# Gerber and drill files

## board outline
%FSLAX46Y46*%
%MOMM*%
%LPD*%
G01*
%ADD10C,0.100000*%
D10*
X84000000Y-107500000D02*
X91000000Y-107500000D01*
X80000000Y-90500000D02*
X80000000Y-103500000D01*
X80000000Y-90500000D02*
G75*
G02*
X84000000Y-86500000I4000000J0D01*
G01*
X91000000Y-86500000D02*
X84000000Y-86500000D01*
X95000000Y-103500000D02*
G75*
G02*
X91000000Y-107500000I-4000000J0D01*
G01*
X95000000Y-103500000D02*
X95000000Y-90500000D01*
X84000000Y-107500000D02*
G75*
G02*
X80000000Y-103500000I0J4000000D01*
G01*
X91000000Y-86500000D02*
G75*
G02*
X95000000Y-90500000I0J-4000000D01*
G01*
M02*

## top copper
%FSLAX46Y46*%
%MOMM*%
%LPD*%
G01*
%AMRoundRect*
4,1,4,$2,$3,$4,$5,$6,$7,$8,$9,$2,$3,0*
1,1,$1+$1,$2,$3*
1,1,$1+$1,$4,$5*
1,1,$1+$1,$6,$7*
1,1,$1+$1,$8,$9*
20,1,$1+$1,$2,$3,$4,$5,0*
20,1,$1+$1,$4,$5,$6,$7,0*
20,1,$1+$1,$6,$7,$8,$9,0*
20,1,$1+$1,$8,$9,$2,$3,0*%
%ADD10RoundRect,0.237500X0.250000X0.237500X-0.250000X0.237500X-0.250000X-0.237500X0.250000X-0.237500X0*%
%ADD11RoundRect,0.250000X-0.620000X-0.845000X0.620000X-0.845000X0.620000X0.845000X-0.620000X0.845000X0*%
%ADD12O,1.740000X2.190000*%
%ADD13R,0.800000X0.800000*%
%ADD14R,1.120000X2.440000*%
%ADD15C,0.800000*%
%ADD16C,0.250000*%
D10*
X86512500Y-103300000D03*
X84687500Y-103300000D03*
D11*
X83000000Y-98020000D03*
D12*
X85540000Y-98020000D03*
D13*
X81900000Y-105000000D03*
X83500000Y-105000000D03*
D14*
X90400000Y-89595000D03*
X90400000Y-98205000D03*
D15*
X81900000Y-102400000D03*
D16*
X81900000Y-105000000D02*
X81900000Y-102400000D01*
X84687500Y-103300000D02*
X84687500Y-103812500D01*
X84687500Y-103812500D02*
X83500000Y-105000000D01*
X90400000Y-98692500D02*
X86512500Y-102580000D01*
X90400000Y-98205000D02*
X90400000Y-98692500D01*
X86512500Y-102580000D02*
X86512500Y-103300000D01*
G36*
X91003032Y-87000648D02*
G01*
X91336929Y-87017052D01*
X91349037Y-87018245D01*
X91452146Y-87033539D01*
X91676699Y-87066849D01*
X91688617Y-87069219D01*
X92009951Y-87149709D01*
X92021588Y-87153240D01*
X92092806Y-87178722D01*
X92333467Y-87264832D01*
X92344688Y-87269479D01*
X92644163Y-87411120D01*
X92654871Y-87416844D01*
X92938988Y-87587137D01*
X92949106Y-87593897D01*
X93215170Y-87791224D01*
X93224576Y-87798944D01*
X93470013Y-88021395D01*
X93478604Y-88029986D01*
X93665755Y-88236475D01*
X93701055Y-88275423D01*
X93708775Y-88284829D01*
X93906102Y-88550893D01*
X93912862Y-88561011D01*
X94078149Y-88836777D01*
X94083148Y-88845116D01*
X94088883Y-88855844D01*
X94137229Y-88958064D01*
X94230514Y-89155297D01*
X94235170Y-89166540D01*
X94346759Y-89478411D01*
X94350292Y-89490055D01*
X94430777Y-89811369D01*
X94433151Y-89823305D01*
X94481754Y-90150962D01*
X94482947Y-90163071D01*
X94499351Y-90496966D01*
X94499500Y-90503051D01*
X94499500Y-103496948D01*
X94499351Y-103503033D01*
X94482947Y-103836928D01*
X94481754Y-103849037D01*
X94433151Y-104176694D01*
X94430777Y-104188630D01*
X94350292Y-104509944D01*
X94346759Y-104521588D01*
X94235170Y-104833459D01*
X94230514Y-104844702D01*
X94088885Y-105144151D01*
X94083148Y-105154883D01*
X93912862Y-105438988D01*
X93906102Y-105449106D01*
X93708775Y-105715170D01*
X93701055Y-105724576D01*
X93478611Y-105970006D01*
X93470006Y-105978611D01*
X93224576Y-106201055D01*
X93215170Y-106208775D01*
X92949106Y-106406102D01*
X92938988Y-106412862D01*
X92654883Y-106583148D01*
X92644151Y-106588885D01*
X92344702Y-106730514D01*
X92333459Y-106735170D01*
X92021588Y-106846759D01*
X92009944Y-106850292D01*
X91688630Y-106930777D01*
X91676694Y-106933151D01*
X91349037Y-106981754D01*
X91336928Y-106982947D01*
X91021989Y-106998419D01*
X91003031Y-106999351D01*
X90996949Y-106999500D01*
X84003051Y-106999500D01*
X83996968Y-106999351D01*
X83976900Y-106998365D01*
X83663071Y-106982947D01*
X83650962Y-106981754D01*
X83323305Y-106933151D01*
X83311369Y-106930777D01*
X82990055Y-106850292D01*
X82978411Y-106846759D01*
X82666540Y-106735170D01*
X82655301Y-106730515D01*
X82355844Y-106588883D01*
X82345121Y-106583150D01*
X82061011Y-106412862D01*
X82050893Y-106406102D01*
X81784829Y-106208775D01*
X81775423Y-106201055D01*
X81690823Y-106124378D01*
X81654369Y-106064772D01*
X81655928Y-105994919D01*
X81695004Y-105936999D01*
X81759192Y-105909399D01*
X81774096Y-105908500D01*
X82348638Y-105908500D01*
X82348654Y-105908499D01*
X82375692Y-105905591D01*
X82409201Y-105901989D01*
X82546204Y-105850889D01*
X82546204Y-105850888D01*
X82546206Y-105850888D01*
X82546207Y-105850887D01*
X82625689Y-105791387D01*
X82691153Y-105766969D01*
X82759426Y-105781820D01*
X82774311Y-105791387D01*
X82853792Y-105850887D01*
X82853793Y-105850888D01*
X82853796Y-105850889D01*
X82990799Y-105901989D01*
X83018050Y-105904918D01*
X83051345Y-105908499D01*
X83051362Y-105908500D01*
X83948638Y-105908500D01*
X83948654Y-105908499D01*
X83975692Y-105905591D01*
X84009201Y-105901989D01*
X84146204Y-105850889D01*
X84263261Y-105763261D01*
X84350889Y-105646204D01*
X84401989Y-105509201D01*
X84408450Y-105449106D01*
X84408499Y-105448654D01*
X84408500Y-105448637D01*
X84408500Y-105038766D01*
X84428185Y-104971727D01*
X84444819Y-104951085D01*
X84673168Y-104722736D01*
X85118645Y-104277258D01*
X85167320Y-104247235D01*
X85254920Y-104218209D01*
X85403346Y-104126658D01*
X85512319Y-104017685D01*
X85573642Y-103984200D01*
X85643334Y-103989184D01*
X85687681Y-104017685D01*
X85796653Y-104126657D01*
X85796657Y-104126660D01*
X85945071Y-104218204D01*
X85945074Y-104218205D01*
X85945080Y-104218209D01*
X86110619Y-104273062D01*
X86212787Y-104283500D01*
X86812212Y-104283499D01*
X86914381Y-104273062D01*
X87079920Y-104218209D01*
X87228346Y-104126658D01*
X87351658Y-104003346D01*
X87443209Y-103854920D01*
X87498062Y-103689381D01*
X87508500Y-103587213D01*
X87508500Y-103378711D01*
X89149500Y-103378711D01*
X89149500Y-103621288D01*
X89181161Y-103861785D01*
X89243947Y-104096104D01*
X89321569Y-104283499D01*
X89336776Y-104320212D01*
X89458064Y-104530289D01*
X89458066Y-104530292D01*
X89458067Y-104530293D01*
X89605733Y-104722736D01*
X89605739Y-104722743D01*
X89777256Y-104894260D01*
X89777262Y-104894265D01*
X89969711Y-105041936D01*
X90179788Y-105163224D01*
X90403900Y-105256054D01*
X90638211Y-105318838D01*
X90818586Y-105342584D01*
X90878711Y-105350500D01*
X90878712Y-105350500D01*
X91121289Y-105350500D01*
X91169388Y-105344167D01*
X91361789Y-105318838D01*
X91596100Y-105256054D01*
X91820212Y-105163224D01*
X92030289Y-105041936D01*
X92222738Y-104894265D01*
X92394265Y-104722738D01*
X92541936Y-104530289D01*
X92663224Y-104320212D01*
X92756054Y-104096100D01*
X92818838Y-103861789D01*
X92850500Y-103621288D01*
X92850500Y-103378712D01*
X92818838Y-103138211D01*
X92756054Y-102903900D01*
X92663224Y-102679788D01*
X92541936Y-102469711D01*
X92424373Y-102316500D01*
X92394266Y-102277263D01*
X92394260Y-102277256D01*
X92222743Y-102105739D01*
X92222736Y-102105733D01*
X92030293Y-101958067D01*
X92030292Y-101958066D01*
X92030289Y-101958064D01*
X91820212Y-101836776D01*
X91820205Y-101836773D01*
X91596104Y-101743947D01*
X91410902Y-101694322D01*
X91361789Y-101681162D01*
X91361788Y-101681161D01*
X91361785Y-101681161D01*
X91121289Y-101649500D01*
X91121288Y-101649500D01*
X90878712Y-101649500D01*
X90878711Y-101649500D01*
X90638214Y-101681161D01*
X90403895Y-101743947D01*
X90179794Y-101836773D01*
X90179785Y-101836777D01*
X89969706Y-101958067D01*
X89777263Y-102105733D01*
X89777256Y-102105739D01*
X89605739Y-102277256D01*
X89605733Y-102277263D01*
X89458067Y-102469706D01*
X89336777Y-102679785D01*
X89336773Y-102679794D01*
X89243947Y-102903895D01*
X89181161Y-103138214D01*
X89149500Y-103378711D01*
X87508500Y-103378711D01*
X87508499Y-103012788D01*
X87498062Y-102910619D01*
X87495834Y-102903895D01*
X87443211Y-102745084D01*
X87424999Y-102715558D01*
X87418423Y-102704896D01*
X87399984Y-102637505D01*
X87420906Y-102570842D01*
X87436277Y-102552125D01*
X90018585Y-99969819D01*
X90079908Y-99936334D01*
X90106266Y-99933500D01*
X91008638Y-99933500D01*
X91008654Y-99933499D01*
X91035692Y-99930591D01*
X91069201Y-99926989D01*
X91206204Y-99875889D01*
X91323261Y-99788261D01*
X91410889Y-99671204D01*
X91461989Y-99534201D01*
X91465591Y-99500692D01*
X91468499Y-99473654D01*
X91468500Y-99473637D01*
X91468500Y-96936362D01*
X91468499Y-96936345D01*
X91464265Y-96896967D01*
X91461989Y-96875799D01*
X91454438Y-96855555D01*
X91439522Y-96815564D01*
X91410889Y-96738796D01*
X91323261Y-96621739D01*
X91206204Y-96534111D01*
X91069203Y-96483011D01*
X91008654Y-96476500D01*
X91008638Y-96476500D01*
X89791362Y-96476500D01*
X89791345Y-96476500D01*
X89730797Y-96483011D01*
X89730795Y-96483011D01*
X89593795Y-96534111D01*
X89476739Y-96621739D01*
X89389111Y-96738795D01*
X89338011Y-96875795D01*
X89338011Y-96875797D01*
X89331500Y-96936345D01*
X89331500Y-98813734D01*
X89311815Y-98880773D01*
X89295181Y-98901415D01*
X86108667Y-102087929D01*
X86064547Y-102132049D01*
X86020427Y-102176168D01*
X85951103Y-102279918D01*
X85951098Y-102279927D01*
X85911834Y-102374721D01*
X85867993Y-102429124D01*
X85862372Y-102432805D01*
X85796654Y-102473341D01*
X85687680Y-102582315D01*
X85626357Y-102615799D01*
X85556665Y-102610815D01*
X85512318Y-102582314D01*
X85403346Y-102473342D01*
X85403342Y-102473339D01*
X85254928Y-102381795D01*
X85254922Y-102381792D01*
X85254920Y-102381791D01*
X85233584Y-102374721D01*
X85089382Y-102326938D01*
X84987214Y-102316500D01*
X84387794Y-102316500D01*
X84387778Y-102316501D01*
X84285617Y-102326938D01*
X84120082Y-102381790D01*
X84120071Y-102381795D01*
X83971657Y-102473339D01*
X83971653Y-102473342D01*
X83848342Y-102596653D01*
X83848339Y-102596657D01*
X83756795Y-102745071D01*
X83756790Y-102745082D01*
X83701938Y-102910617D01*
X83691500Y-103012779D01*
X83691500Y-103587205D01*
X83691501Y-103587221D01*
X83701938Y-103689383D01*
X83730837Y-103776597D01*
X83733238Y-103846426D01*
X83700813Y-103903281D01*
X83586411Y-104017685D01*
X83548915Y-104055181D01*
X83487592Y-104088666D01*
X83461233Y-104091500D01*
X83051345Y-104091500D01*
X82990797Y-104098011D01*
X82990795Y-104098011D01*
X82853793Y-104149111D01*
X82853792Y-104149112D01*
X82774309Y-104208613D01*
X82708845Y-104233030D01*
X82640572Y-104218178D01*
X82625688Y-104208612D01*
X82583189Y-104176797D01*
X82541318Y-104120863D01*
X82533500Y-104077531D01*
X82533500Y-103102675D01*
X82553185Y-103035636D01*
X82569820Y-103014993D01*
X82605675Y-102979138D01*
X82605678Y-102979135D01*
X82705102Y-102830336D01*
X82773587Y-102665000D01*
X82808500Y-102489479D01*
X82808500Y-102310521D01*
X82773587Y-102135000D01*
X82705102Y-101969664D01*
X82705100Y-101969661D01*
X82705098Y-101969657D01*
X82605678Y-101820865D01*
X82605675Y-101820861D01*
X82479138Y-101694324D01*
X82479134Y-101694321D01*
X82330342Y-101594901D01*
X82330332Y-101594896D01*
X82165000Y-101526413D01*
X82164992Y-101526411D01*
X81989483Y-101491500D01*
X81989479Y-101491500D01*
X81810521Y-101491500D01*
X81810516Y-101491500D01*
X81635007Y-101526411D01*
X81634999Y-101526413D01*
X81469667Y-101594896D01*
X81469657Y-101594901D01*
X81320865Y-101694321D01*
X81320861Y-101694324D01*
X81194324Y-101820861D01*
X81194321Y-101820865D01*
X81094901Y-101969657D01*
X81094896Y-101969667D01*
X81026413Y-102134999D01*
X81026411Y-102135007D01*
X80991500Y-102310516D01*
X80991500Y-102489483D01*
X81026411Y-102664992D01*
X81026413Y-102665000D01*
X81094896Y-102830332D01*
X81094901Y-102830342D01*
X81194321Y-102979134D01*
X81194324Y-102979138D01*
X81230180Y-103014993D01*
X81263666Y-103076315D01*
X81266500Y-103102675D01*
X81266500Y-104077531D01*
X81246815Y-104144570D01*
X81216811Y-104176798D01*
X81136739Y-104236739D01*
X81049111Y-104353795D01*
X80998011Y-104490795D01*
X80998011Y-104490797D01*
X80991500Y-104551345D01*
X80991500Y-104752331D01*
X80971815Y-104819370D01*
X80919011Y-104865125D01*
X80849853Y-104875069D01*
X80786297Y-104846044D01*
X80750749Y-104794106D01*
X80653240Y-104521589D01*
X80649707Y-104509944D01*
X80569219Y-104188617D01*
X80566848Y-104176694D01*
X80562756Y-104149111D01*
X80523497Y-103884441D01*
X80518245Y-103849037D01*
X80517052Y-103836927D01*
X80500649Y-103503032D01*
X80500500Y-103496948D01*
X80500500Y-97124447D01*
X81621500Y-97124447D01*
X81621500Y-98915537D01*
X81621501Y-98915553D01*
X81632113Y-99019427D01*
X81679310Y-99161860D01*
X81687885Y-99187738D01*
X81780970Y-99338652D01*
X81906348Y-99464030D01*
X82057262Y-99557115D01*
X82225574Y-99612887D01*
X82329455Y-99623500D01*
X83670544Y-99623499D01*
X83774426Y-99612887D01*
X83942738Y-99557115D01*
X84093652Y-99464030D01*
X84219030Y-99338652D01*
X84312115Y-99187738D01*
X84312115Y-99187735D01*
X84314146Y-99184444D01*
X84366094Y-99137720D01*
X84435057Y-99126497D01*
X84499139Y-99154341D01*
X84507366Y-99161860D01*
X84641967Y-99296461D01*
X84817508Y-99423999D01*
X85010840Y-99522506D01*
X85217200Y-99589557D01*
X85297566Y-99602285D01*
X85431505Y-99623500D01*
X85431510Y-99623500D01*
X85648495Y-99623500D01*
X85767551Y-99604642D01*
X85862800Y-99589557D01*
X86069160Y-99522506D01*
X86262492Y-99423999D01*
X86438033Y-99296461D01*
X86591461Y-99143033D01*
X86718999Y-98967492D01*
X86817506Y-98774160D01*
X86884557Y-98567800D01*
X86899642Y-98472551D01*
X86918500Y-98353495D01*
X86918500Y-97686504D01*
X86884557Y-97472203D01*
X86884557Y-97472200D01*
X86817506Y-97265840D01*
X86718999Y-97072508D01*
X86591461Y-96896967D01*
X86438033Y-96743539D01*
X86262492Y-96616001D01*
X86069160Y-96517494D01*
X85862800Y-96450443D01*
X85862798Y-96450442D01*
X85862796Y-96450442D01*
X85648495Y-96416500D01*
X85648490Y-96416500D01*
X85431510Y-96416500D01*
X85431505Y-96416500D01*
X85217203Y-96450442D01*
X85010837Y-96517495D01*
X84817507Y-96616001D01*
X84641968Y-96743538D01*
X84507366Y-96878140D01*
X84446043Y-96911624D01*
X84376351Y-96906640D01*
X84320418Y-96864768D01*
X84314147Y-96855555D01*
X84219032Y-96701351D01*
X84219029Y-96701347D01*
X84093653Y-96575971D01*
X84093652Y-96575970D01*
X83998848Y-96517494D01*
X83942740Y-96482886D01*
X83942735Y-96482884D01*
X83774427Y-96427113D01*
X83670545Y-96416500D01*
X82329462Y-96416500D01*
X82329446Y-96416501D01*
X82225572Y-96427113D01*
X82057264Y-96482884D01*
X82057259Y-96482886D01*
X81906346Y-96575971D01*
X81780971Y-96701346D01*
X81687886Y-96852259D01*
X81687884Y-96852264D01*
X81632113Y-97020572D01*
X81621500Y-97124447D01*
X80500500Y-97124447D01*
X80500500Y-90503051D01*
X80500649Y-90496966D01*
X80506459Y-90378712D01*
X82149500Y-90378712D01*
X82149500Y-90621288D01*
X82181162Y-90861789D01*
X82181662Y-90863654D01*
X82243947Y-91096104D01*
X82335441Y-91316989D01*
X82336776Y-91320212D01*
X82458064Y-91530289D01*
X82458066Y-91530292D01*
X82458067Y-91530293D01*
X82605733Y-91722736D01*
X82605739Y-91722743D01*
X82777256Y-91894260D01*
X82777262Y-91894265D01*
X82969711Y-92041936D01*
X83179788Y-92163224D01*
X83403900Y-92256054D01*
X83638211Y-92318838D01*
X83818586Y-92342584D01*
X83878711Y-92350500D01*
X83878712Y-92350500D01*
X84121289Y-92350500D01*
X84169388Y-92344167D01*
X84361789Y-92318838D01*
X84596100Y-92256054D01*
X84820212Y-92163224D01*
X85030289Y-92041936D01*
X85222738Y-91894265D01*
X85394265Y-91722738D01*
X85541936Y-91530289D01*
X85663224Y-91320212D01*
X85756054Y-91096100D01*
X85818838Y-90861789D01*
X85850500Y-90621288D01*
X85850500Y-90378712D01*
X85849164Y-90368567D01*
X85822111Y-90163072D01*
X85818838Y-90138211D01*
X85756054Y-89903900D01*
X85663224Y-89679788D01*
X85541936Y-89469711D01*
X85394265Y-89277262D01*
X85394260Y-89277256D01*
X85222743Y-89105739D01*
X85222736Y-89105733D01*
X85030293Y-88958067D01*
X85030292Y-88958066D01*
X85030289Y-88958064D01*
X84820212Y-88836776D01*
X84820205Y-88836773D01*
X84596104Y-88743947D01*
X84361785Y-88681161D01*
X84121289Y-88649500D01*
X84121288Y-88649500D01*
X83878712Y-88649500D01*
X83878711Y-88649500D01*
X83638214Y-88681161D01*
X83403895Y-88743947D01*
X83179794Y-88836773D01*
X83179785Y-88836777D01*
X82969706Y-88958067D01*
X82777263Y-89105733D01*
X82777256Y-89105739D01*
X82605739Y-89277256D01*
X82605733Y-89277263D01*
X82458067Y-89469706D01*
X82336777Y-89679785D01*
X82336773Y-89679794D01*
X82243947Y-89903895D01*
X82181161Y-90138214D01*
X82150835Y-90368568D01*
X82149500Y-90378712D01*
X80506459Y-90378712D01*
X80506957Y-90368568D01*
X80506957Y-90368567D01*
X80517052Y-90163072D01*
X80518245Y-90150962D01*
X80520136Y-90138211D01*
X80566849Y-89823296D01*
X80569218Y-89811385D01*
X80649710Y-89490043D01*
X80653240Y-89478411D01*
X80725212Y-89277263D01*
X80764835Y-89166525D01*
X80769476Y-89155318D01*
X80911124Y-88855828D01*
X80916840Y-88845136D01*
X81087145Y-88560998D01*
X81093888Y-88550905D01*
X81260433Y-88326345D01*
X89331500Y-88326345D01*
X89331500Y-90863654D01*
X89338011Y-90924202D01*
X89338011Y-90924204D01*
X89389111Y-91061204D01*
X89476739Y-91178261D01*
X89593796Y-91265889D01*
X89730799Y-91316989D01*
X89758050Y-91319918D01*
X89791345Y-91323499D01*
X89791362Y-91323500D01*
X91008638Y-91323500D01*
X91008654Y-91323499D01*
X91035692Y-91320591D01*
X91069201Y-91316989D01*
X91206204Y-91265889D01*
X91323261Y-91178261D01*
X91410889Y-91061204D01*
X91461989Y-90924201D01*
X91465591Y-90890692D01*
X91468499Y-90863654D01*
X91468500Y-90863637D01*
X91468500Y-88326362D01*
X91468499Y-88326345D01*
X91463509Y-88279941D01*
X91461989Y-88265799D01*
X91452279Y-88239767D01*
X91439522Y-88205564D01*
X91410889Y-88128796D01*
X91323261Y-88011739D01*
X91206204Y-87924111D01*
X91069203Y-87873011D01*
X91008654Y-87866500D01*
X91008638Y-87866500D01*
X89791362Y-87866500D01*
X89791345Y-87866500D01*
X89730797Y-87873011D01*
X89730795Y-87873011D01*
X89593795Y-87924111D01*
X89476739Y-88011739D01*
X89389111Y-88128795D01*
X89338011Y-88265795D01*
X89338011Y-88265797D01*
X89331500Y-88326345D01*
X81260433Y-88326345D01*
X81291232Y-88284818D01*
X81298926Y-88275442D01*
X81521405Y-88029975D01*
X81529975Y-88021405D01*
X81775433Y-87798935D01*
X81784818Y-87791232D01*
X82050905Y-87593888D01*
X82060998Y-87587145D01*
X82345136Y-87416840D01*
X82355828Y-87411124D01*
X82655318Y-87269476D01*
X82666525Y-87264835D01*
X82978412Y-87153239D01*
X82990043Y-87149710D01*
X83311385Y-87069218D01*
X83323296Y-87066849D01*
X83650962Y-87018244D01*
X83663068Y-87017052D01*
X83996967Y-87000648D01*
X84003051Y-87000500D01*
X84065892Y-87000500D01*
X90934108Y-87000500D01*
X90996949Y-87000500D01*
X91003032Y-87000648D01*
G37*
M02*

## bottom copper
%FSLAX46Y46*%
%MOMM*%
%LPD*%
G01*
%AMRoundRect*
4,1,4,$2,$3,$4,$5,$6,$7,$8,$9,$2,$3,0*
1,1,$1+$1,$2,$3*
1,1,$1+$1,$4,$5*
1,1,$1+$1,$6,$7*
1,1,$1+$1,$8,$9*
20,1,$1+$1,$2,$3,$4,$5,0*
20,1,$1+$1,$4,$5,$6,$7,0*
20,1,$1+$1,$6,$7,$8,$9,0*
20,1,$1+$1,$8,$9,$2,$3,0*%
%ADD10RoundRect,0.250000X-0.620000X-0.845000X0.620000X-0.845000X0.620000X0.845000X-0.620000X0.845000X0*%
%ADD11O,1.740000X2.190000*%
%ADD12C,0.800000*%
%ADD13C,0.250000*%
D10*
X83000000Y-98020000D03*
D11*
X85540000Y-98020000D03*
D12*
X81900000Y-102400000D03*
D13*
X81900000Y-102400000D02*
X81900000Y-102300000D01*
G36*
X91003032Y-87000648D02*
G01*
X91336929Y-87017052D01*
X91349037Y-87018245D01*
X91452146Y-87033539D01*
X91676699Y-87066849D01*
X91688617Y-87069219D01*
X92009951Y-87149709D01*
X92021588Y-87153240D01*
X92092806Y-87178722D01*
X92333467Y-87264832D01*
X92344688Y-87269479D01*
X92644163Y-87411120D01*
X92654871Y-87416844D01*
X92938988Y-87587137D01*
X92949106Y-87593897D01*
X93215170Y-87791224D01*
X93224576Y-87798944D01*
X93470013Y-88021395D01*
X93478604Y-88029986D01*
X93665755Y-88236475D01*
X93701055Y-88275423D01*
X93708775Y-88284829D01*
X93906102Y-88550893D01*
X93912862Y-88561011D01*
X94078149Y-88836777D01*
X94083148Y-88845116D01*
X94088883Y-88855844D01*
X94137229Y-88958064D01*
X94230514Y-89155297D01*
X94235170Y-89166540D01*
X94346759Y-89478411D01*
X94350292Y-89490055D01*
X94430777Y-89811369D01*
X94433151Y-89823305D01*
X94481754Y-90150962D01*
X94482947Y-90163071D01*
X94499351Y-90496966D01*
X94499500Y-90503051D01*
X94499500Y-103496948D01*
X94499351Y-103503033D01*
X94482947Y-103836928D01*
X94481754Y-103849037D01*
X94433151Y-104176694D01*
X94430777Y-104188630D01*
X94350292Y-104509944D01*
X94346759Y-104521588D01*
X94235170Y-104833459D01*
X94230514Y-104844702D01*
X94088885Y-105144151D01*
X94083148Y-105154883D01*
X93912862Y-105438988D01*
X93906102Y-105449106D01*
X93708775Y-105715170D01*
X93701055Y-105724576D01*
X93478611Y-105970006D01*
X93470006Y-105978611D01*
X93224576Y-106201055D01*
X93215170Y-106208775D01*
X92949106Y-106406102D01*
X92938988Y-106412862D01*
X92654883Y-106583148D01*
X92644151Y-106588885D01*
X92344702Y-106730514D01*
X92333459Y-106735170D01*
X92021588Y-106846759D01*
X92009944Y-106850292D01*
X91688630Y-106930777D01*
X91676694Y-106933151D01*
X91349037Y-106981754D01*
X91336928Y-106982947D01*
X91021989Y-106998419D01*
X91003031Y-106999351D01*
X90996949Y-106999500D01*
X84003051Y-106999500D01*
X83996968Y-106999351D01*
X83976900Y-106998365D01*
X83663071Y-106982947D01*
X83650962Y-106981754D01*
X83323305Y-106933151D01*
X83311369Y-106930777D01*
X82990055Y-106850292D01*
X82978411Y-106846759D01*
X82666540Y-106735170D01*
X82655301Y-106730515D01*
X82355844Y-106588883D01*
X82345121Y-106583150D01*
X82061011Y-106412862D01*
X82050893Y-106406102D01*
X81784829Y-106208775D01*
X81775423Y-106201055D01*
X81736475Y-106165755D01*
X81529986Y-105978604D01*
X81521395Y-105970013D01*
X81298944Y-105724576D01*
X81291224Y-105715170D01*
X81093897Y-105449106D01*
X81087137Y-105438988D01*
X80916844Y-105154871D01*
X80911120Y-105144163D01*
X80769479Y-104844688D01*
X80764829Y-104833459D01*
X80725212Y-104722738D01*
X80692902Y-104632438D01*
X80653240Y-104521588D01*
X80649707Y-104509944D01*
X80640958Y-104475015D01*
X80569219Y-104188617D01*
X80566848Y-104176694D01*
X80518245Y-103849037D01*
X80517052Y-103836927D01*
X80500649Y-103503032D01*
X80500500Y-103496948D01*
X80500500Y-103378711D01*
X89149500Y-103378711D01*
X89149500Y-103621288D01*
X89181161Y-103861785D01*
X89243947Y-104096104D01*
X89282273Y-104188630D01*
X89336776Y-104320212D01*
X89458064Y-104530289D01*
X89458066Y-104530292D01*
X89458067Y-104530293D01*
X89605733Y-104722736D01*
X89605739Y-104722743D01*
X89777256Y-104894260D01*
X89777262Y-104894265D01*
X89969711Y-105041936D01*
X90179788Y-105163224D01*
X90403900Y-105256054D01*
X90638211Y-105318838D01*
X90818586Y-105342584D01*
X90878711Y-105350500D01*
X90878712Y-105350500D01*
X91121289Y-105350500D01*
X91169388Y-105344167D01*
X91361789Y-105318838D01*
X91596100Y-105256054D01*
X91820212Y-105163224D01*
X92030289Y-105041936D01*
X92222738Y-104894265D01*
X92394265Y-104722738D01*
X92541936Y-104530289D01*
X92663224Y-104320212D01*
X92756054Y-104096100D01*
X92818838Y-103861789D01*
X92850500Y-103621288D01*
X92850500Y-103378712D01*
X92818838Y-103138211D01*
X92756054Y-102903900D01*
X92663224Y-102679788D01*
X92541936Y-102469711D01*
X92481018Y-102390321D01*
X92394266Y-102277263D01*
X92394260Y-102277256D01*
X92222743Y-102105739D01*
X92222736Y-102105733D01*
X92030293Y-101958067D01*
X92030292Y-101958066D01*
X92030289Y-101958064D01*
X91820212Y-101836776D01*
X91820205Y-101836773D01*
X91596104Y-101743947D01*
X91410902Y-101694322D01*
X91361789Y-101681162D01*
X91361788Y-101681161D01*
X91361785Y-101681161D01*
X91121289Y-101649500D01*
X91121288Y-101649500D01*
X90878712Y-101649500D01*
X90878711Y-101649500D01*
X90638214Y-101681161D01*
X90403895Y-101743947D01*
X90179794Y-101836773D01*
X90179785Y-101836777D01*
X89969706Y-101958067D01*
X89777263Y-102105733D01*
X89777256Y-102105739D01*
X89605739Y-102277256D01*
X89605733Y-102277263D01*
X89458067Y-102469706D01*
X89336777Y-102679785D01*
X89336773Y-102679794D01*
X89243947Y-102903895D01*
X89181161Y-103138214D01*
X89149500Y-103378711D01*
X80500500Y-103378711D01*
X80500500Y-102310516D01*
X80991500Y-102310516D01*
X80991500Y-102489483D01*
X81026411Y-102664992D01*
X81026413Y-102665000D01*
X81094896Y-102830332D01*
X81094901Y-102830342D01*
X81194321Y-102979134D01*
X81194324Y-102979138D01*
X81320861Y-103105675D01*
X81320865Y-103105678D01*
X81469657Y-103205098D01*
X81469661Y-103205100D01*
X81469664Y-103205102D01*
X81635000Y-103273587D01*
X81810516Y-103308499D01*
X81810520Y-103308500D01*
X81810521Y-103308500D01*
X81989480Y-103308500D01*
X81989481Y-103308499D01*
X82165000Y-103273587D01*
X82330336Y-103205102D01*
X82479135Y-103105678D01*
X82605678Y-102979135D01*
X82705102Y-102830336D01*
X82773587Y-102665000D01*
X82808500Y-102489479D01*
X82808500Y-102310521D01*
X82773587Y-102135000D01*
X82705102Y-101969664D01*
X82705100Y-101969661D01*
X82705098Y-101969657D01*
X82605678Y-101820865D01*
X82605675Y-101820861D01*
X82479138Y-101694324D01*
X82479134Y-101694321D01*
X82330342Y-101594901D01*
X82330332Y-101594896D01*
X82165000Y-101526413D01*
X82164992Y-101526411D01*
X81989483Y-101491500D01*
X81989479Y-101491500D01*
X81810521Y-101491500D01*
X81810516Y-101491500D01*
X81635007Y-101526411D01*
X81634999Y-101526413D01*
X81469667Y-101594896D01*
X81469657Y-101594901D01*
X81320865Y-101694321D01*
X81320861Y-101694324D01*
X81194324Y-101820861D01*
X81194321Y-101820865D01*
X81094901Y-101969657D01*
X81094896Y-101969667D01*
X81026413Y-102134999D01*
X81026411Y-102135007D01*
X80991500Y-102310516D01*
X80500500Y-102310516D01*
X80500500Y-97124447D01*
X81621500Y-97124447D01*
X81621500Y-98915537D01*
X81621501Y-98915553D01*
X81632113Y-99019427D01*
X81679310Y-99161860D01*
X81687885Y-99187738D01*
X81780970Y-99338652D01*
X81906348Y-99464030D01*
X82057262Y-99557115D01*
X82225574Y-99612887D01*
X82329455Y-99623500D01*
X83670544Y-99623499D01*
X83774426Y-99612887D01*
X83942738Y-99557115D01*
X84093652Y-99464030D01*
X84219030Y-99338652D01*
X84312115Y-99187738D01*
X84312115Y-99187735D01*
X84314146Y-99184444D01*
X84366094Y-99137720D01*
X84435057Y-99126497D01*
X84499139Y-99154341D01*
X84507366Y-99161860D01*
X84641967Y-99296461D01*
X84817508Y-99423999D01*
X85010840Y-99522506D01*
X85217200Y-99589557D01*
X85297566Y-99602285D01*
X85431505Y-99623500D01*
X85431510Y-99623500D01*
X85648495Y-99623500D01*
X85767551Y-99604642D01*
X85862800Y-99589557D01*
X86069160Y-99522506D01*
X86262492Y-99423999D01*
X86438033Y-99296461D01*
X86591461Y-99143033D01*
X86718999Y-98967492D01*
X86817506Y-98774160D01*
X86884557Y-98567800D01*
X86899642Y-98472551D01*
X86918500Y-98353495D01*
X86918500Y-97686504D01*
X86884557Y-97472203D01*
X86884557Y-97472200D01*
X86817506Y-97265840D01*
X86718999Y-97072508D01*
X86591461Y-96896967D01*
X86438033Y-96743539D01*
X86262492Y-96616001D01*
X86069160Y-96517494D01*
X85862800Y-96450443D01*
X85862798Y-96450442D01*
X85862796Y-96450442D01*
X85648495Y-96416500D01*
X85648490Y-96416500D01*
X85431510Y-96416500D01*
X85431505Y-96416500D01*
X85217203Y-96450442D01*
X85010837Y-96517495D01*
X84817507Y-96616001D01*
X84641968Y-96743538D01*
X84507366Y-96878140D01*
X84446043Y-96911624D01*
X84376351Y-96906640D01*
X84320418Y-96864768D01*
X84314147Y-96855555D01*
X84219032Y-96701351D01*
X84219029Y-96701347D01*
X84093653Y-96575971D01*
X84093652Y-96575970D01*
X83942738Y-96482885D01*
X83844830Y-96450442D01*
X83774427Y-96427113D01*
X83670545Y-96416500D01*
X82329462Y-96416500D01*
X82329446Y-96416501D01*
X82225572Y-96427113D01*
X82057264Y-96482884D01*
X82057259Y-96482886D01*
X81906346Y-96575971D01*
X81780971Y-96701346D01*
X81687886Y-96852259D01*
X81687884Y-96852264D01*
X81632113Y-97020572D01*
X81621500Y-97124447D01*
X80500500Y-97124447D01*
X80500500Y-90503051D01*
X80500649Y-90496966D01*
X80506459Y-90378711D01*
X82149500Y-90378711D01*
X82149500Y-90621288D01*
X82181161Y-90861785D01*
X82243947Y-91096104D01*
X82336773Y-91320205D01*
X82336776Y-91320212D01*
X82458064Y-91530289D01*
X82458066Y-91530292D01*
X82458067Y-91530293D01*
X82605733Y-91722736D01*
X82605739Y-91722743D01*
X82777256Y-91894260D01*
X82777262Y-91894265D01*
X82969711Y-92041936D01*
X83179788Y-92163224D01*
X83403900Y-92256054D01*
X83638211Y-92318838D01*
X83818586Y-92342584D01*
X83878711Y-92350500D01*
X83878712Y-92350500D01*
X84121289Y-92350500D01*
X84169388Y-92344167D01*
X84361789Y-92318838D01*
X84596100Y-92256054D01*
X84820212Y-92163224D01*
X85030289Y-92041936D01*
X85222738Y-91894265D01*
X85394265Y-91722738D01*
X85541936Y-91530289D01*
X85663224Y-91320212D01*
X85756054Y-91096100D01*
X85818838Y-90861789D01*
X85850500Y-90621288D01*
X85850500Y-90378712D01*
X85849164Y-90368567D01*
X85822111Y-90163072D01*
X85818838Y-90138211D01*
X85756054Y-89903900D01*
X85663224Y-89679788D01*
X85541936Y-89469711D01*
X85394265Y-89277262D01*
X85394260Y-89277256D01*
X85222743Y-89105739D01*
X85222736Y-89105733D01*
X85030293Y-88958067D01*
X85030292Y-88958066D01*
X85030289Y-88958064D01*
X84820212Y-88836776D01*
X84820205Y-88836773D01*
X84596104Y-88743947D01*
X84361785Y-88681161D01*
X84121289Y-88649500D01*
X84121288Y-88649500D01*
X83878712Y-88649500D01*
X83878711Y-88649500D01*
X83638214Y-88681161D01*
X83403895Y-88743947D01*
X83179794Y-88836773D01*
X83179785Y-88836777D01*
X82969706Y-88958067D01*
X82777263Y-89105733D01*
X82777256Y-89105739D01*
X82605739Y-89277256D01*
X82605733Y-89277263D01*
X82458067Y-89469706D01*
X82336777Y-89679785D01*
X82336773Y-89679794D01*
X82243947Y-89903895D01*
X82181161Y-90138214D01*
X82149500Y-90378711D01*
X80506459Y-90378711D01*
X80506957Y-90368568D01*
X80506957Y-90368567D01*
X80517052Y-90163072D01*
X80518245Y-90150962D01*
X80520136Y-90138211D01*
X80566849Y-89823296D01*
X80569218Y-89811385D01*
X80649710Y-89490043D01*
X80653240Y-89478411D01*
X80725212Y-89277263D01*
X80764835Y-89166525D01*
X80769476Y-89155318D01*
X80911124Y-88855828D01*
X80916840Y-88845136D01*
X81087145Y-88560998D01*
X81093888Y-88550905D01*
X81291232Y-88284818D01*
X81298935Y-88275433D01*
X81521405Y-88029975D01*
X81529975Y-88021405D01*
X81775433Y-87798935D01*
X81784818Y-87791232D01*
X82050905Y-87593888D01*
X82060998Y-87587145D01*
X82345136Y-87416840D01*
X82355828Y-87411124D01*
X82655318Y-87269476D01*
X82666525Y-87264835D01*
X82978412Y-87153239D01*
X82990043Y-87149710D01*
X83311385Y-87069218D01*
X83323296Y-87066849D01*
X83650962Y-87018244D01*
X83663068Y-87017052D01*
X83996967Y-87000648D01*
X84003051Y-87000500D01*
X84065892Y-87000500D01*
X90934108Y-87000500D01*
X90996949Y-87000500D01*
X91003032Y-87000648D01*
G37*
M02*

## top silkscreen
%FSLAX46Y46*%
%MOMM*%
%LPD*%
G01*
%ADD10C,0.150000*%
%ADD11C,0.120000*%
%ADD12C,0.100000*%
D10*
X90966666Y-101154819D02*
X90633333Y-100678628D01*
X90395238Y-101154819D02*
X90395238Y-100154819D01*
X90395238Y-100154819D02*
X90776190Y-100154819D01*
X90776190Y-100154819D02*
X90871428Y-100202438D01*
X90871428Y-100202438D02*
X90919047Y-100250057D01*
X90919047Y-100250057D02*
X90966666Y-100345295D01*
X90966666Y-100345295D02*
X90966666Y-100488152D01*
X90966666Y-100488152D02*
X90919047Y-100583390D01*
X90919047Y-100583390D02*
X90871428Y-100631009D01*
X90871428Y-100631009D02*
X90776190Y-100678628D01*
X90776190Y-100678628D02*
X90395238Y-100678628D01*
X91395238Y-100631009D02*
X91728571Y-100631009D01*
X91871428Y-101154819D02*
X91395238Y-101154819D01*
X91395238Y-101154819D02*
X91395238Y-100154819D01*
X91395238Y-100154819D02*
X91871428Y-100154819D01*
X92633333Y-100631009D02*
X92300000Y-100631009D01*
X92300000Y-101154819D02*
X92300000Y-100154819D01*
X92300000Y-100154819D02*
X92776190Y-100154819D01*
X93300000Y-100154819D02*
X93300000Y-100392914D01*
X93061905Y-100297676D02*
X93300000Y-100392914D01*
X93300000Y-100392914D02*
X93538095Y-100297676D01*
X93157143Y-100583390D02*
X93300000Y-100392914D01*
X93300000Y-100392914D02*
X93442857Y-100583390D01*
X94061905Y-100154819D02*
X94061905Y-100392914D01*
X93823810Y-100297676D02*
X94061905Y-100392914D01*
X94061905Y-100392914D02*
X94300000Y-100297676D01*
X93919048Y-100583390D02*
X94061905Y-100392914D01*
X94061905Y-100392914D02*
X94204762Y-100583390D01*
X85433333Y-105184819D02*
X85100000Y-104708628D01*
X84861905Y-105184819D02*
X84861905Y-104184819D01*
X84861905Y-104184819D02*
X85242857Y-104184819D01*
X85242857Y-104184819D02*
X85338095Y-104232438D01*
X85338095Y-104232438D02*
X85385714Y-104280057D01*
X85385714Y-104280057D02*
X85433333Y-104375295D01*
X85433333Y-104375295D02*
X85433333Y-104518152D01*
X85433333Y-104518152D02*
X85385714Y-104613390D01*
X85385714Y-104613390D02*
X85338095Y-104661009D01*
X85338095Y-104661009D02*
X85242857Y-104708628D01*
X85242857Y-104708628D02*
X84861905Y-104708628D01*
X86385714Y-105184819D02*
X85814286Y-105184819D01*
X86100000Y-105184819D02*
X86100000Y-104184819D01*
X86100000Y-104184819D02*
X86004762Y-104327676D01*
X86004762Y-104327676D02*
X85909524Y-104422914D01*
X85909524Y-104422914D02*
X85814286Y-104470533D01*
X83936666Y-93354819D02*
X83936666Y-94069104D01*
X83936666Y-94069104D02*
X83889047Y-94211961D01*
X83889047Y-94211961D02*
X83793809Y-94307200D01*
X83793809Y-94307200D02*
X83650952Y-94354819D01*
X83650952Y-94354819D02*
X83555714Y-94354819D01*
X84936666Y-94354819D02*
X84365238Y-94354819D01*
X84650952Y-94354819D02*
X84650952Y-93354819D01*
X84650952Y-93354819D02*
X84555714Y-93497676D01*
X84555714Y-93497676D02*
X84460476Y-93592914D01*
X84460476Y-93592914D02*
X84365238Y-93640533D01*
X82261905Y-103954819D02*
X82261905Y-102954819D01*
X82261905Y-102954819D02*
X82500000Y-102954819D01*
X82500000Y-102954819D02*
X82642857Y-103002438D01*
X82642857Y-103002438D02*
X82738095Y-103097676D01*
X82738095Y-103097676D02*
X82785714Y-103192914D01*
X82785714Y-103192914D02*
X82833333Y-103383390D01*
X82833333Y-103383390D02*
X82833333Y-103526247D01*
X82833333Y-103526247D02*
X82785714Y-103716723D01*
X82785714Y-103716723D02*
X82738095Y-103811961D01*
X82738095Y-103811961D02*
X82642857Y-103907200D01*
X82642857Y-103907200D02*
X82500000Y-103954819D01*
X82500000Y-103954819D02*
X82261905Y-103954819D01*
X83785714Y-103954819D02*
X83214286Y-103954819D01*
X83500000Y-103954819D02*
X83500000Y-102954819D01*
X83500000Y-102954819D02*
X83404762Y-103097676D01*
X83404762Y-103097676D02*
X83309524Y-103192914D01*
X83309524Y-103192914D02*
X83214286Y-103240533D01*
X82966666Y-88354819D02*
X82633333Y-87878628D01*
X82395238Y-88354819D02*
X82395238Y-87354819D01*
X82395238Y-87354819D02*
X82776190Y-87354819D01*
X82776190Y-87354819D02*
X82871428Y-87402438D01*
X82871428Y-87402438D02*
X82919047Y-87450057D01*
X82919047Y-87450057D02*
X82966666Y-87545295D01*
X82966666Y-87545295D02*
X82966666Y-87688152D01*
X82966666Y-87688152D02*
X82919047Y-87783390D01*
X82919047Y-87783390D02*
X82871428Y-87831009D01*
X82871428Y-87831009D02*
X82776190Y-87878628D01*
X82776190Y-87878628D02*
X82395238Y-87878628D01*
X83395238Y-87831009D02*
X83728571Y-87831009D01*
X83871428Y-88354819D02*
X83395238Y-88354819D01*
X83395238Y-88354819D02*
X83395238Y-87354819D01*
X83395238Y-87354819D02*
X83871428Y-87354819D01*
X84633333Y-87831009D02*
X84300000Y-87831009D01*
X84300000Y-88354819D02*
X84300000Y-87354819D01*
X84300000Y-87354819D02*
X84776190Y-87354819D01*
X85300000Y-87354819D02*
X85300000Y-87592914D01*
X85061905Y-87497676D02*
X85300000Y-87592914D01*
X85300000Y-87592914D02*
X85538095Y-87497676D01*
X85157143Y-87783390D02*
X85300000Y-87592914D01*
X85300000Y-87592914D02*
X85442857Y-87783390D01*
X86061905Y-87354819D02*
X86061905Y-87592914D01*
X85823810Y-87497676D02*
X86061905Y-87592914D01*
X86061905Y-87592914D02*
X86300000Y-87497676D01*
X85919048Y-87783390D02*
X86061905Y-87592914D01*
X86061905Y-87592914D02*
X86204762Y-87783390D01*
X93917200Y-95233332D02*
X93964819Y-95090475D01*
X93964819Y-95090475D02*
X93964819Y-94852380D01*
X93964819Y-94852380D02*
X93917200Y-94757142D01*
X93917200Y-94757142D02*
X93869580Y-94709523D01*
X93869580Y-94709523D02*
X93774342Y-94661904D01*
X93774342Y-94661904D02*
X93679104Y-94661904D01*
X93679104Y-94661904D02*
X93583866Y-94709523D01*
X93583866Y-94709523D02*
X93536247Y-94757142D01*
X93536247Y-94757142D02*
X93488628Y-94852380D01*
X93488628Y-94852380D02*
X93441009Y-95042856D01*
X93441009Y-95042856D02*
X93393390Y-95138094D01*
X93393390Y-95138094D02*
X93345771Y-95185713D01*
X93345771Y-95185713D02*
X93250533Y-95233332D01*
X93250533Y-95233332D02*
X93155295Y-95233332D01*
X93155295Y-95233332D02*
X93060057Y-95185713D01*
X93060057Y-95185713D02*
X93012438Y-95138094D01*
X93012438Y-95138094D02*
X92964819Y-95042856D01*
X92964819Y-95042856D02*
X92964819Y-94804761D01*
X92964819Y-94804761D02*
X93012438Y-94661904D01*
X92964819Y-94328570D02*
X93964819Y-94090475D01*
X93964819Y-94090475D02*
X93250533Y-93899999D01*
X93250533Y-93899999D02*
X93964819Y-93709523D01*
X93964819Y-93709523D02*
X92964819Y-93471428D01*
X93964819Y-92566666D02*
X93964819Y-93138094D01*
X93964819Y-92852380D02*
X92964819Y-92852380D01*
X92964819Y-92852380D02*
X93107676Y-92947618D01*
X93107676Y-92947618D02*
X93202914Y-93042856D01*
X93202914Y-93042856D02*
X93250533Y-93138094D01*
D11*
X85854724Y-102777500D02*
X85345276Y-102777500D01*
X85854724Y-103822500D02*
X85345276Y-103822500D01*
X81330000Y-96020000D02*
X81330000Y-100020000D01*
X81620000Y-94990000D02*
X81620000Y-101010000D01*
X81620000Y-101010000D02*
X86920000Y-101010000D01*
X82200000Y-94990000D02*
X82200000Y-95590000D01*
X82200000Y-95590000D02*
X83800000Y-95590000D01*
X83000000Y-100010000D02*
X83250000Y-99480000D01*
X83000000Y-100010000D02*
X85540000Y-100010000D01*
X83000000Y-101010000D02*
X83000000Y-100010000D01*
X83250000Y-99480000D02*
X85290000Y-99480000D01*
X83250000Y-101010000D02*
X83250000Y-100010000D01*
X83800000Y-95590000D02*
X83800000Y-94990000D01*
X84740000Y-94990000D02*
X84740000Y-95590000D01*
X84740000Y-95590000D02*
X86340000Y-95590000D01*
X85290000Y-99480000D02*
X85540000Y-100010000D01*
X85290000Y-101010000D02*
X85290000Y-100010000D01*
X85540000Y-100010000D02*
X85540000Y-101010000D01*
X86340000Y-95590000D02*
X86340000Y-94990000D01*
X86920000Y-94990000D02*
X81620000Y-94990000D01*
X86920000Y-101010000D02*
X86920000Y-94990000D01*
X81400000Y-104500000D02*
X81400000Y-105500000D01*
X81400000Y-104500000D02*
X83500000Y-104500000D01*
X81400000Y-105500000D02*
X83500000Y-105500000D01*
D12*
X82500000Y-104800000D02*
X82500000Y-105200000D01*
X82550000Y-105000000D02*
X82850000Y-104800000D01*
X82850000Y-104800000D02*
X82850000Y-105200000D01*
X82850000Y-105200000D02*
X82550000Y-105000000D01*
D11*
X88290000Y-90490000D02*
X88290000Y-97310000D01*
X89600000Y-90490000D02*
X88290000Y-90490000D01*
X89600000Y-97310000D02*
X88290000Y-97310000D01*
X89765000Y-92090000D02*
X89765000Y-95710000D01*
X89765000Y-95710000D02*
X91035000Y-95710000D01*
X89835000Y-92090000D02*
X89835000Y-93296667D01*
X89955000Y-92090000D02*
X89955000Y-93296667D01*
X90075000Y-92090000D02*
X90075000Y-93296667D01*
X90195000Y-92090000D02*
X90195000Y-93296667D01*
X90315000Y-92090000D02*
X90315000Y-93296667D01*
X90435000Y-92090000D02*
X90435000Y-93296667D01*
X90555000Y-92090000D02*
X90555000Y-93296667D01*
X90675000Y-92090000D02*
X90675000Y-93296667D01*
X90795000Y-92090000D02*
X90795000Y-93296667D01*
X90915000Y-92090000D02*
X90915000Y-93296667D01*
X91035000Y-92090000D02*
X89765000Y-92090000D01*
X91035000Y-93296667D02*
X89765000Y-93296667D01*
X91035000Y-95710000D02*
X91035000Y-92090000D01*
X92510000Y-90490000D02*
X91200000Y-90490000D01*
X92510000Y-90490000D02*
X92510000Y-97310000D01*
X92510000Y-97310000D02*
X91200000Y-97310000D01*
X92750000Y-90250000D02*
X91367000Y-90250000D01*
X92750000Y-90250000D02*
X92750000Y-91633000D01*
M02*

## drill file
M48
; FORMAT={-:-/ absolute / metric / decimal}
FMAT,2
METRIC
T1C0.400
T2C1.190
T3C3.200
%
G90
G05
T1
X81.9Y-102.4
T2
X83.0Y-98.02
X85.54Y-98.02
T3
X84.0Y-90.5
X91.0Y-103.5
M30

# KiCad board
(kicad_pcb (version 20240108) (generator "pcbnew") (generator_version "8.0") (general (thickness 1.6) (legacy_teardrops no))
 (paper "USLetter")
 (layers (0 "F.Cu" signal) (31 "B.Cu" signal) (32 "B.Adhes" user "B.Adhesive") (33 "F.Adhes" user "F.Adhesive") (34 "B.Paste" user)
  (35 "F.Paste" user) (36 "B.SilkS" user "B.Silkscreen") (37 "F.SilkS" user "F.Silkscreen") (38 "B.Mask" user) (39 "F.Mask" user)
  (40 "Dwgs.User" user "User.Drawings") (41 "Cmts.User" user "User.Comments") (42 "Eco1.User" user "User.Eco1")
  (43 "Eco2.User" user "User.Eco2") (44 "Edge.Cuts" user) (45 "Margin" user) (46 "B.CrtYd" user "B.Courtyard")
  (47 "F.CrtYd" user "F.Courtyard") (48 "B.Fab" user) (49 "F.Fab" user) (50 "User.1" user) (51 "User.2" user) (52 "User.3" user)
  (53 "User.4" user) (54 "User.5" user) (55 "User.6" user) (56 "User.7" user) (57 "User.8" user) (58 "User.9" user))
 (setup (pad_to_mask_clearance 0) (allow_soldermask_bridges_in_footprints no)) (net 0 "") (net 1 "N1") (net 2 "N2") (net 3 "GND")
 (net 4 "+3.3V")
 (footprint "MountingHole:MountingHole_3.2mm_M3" (layer "F.Cu") (at 91 103.5)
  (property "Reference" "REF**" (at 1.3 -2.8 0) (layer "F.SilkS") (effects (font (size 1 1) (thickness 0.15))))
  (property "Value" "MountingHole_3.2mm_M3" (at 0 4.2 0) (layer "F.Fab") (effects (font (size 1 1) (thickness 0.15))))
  (pad "" np_thru_hole circle (at 0 0) (size 3.2 3.2) (drill 3.2) (layers "*.Cu" "*.Mask")))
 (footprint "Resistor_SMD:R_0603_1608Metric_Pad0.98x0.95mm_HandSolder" (layer "F.Cu") (at 85.6 103.3 180)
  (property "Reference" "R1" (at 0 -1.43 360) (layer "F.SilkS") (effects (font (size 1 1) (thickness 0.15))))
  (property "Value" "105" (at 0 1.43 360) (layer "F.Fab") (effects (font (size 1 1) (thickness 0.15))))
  (fp_line (start -0.254724 0.5225) (end 0.254724 0.5225) (stroke (width 0.12) (type solid)) (layer "F.SilkS"))
  (fp_line (start -0.254724 -0.5225) (end 0.254724 -0.5225) (stroke (width 0.12) (type solid)) (layer "F.SilkS"))
  (pad "1" smd roundrect (at -0.9125 0 180) (size 0.975 0.95) (layers "F.Cu" "F.Paste" "F.Mask") (roundrect_rratio 0.25) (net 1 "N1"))
  (pad "2" smd roundrect (at 0.9125 0 180) (size 0.975 0.95) (layers "F.Cu" "F.Paste" "F.Mask") (roundrect_rratio 0.25) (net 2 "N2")))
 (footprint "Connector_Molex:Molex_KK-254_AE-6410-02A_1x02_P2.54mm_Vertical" (layer "F.Cu") (at 83 98.02)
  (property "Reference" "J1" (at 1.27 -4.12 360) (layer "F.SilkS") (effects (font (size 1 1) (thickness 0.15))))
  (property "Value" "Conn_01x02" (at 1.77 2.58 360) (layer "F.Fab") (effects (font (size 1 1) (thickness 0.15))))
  (fp_line (start -1.67 -2) (end -1.67 2) (stroke (width 0.12) (type solid)) (layer "F.SilkS"))
  (fp_line (start -1.38 -3.03) (end -1.38 2.99) (stroke (width 0.12) (type solid)) (layer "F.SilkS"))
  (fp_line (start -1.38 2.99) (end 3.92 2.99) (stroke (width 0.12) (type solid)) (layer "F.SilkS"))
  (fp_line (start -0.8 -3.03) (end -0.8 -2.43) (stroke (width 0.12) (type solid)) (layer "F.SilkS"))
  (fp_line (start -0.8 -2.43) (end 0.8 -2.43) (stroke (width 0.12) (type solid)) (layer "F.SilkS"))
  (fp_line (start 0 1.99) (end 0.25 1.46) (stroke (width 0.12) (type solid)) (layer "F.SilkS"))
  (fp_line (start 0 1.99) (end 2.54 1.99) (stroke (width 0.12) (type solid)) (layer "F.SilkS"))
  (fp_line (start 0 2.99) (end 0 1.99) (stroke (width 0.12) (type solid)) (layer "F.SilkS"))
  (fp_line (start 0.25 1.46) (end 2.29 1.46) (stroke (width 0.12) (type solid)) (layer "F.SilkS"))
  (fp_line (start 0.25 2.99) (end 0.25 1.99) (stroke (width 0.12) (type solid)) (layer "F.SilkS"))
  (fp_line (start 0.8 -2.43) (end 0.8 -3.03) (stroke (width 0.12) (type solid)) (layer "F.SilkS"))
  (fp_line (start 1.74 -3.03) (end 1.74 -2.43) (stroke (width 0.12) (type solid)) (layer "F.SilkS"))
  (fp_line (start 1.74 -2.43) (end 3.34 -2.43) (stroke (width 0.12) (type solid)) (layer "F.SilkS"))
  (fp_line (start 2.29 1.46) (end 2.54 1.99) (stroke (width 0.12) (type solid)) (layer "F.SilkS"))
  (fp_line (start 2.29 2.99) (end 2.29 1.99) (stroke (width 0.12) (type solid)) (layer "F.SilkS"))
  (fp_line (start 2.54 1.99) (end 2.54 2.99) (stroke (width 0.12) (type solid)) (layer "F.SilkS"))
  (fp_line (start 3.34 -2.43) (end 3.34 -3.03) (stroke (width 0.12) (type solid)) (layer "F.SilkS"))
  (fp_line (start 3.92 -3.03) (end -1.38 -3.03) (stroke (width 0.12) (type solid)) (layer "F.SilkS"))
  (fp_line (start 3.92 2.99) (end 3.92 -3.03) (stroke (width 0.12) (type solid)) (layer "F.SilkS"))
  (pad "1" thru_hole roundrect (at 0 0) (size 1.74 2.19) (drill 1.19) (layers "*.Cu" "*.Mask") (remove_unused_layers no)
   (roundrect_rratio 0.143678) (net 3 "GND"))
  (pad "2" thru_hole oval (at 2.54 0) (size 1.74 2.19) (drill 1.19) (layers "*.Cu" "*.Mask") (remove_unused_layers no) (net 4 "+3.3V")))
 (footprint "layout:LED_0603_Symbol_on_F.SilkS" (layer "F.Cu") (at 82.7 105)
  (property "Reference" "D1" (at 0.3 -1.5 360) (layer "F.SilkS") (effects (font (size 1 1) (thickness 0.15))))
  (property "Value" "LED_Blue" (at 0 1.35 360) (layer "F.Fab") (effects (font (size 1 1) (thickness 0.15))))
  (fp_line (start -1.3 -0.5) (end -1.3 0.5) (stroke (width 0.12) (type solid)) (layer "F.SilkS"))
  (fp_line (start -1.3 -0.5) (end 0.8 -0.5) (stroke (width 0.12) (type solid)) (layer "F.SilkS"))
  (fp_line (start -1.3 0.5) (end 0.8 0.5) (stroke (width 0.12) (type solid)) (layer "F.SilkS"))
  (fp_line (start -0.2 -0.2) (end -0.2 0.2) (stroke (width 0.1) (type solid)) (layer "F.SilkS"))
  (fp_line (start -0.15 0) (end 0.15 -0.2) (stroke (width 0.1) (type solid)) (layer "F.SilkS"))
  (fp_line (start 0.15 -0.2) (end 0.15 0.2) (stroke (width 0.1) (type solid)) (layer "F.SilkS"))
  (fp_line (start 0.15 0.2) (end -0.15 0) (stroke (width 0.1) (type solid)) (layer "F.SilkS"))
  (pad "1" smd rect (at -0.8 0 180) (size 0.8 0.8) (layers "F.Cu" "F.Paste" "F.Mask") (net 3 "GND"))
  (pad "2" smd rect (at 0.8 0 180) (size 0.8 0.8) (layers "F.Cu" "F.Paste" "F.Mask") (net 2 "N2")))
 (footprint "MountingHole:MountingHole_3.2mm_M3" (layer "F.Cu") (at 84 90.5)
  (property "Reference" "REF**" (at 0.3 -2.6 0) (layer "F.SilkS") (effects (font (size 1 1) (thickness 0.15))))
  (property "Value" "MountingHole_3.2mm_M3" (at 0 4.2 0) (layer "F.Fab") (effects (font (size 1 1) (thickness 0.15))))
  (pad "" np_thru_hole circle (at 0 0) (size 3.2 3.2) (drill 3.2) (layers "*.Cu" "*.Mask")))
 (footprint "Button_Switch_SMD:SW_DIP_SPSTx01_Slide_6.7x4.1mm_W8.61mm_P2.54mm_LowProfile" (layer "F.Cu") (at 90.4 93.9 -90)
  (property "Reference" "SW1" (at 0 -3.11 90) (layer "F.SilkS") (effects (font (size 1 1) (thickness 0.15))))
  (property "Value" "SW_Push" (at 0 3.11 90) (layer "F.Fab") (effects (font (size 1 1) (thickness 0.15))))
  (fp_line (start -3.41 2.11) (end 3.41 2.11) (stroke (width 0.12) (type solid)) (layer "F.SilkS"))
  (fp_line (start -3.41 0.8) (end -3.41 2.11) (stroke (width 0.12) (type solid)) (layer "F.SilkS"))
  (fp_line (start 3.41 0.8) (end 3.41 2.11) (stroke (width 0.12) (type solid)) (layer "F.SilkS"))
  (fp_line (start -1.81 0.635) (end 1.81 0.635) (stroke (width 0.12) (type solid)) (layer "F.SilkS"))
  (fp_line (start 1.81 0.635) (end 1.81 -0.635) (stroke (width 0.12) (type solid)) (layer "F.SilkS"))
  (fp_line (start -1.81 0.565) (end -0.603333 0.565) (stroke (width 0.12) (type solid)) (layer "F.SilkS"))
  (fp_line (start -1.81 0.445) (end -0.603333 0.445) (stroke (width 0.12) (type solid)) (layer "F.SilkS"))
  (fp_line (start -1.81 0.325) (end -0.603333 0.325) (stroke (width 0.12) (type solid)) (layer "F.SilkS"))
  (fp_line (start -1.81 0.205) (end -0.603333 0.205) (stroke (width 0.12) (type solid)) (layer "F.SilkS"))
  (fp_line (start -1.81 0.085) (end -0.603333 0.085) (stroke (width 0.12) (type solid)) (layer "F.SilkS"))
  (fp_line (start -1.81 -0.035) (end -0.603333 -0.035) (stroke (width 0.12) (type solid)) (layer "F.SilkS"))
  (fp_line (start -1.81 -0.155) (end -0.603333 -0.155) (stroke (width 0.12) (type solid)) (layer "F.SilkS"))
  (fp_line (start -1.81 -0.275) (end -0.603333 -0.275) (stroke (width 0.12) (type solid)) (layer "F.SilkS"))
  (fp_line (start -1.81 -0.395) (end -0.603333 -0.395) (stroke (width 0.12) (type solid)) (layer "F.SilkS"))
  (fp_line (start -1.81 -0.515) (end -0.603333 -0.515) (stroke (width 0.12) (type solid)) (layer "F.SilkS"))
  (fp_line (start -1.81 -0.635) (end -1.81 0.635) (stroke (width 0.12) (type solid)) (layer "F.SilkS"))
  (fp_line (start -0.603333 -0.635) (end -0.603333 0.635) (stroke (width 0.12) (type solid)) (layer "F.SilkS"))
  (fp_line (start 1.81 -0.635) (end -1.81 -0.635) (stroke (width 0.12) (type solid)) (layer "F.SilkS"))
  (fp_line (start -3.41 -2.11) (end -3.41 -0.8) (stroke (width 0.12) (type solid)) (layer "F.SilkS"))
  (fp_line (start -3.41 -2.11) (end 3.41 -2.11) (stroke (width 0.12) (type solid)) (layer "F.SilkS"))
  (fp_line (start 3.41 -2.11) (end 3.41 -0.8) (stroke (width 0.12) (type solid)) (layer "F.SilkS"))
  (fp_line (start -3.65 -2.35) (end -3.65 -0.967) (stroke (width 0.12) (type solid)) (layer "F.SilkS"))
  (fp_line (start -3.65 -2.35) (end -2.267 -2.35) (stroke (width 0.12) (type solid)) (layer "F.SilkS"))
  (pad "1" smd rect (at -4.305 0 270) (size 2.44 1.12) (layers "F.Cu" "F.Paste" "F.Mask") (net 4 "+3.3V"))
  (pad "2" smd rect (at 4.305 0 270) (size 2.44 1.12) (layers "F.Cu" "F.Paste" "F.Mask") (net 1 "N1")))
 (gr_line (start 84 107.5) (end 91 107.5) (stroke (width 0.1) (type default)) (layer "Edge.Cuts"))
 (gr_line (start 80 90.5) (end 80 103.5) (stroke (width 0.1) (type default)) (layer "Edge.Cuts"))
 (gr_arc (start 80 90.5) (mid 81.171573 87.671573) (end 84 86.5) (stroke (width 0.1) (type default)) (layer "Edge.Cuts"))
 (gr_line (start 91 86.5) (end 84 86.5) (stroke (width 0.1) (type default)) (layer "Edge.Cuts"))
 (gr_arc (start 95 103.5) (mid 93.828427 106.328427) (end 91 107.5) (stroke (width 0.1) (type default)) (layer "Edge.Cuts"))
 (gr_line (start 95 103.5) (end 95 90.5) (stroke (width 0.1) (type default)) (layer "Edge.Cuts"))
 (gr_arc (start 84 107.5) (mid 81.171573 106.328427) (end 80 103.5) (stroke (width 0.1) (type default)) (layer "Edge.Cuts"))
 (gr_arc (start 91 86.5) (mid 93.828427 87.671573) (end 95 90.5) (stroke (width 0.1) (type default)) (layer "Edge.Cuts"))
 (segment (start 81.9 105) (end 81.9 102.4) (width 0.25) (layer "F.Cu") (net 3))
 (via (at 81.9 102.4) (size 0.8) (drill 0.4) (layers "F.Cu" "B.Cu") (free yes) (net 3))
 (segment (start 81.9 102.4) (end 81.9 102.3) (width 0.25) (layer "B.Cu") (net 3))
 (segment (start 84.6875 103.3) (end 84.6875 103.8125) (width 0.25) (layer "F.Cu") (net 2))
 (segment (start 84.6875 103.8125) (end 83.5 105) (width 0.25) (layer "F.Cu") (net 2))
 (segment (start 90.4 98.6925) (end 86.5125 102.58) (width 0.25) (layer "F.Cu") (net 1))
 (segment (start 90.4 98.205) (end 90.4 98.6925) (width 0.25) (layer "F.Cu") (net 1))
 (segment (start 86.5125 102.58) (end 86.5125 103.3) (width 0.25) (layer "F.Cu") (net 1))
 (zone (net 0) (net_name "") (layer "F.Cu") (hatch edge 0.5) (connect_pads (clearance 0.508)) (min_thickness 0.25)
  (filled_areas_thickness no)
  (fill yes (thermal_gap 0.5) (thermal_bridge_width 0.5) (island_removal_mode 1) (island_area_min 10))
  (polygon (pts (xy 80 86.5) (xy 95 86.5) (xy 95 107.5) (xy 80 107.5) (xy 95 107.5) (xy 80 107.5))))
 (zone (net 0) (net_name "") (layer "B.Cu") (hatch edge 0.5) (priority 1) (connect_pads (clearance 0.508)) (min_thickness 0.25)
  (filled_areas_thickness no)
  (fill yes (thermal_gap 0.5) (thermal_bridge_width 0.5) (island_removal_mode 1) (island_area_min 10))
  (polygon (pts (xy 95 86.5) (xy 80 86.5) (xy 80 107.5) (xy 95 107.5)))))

